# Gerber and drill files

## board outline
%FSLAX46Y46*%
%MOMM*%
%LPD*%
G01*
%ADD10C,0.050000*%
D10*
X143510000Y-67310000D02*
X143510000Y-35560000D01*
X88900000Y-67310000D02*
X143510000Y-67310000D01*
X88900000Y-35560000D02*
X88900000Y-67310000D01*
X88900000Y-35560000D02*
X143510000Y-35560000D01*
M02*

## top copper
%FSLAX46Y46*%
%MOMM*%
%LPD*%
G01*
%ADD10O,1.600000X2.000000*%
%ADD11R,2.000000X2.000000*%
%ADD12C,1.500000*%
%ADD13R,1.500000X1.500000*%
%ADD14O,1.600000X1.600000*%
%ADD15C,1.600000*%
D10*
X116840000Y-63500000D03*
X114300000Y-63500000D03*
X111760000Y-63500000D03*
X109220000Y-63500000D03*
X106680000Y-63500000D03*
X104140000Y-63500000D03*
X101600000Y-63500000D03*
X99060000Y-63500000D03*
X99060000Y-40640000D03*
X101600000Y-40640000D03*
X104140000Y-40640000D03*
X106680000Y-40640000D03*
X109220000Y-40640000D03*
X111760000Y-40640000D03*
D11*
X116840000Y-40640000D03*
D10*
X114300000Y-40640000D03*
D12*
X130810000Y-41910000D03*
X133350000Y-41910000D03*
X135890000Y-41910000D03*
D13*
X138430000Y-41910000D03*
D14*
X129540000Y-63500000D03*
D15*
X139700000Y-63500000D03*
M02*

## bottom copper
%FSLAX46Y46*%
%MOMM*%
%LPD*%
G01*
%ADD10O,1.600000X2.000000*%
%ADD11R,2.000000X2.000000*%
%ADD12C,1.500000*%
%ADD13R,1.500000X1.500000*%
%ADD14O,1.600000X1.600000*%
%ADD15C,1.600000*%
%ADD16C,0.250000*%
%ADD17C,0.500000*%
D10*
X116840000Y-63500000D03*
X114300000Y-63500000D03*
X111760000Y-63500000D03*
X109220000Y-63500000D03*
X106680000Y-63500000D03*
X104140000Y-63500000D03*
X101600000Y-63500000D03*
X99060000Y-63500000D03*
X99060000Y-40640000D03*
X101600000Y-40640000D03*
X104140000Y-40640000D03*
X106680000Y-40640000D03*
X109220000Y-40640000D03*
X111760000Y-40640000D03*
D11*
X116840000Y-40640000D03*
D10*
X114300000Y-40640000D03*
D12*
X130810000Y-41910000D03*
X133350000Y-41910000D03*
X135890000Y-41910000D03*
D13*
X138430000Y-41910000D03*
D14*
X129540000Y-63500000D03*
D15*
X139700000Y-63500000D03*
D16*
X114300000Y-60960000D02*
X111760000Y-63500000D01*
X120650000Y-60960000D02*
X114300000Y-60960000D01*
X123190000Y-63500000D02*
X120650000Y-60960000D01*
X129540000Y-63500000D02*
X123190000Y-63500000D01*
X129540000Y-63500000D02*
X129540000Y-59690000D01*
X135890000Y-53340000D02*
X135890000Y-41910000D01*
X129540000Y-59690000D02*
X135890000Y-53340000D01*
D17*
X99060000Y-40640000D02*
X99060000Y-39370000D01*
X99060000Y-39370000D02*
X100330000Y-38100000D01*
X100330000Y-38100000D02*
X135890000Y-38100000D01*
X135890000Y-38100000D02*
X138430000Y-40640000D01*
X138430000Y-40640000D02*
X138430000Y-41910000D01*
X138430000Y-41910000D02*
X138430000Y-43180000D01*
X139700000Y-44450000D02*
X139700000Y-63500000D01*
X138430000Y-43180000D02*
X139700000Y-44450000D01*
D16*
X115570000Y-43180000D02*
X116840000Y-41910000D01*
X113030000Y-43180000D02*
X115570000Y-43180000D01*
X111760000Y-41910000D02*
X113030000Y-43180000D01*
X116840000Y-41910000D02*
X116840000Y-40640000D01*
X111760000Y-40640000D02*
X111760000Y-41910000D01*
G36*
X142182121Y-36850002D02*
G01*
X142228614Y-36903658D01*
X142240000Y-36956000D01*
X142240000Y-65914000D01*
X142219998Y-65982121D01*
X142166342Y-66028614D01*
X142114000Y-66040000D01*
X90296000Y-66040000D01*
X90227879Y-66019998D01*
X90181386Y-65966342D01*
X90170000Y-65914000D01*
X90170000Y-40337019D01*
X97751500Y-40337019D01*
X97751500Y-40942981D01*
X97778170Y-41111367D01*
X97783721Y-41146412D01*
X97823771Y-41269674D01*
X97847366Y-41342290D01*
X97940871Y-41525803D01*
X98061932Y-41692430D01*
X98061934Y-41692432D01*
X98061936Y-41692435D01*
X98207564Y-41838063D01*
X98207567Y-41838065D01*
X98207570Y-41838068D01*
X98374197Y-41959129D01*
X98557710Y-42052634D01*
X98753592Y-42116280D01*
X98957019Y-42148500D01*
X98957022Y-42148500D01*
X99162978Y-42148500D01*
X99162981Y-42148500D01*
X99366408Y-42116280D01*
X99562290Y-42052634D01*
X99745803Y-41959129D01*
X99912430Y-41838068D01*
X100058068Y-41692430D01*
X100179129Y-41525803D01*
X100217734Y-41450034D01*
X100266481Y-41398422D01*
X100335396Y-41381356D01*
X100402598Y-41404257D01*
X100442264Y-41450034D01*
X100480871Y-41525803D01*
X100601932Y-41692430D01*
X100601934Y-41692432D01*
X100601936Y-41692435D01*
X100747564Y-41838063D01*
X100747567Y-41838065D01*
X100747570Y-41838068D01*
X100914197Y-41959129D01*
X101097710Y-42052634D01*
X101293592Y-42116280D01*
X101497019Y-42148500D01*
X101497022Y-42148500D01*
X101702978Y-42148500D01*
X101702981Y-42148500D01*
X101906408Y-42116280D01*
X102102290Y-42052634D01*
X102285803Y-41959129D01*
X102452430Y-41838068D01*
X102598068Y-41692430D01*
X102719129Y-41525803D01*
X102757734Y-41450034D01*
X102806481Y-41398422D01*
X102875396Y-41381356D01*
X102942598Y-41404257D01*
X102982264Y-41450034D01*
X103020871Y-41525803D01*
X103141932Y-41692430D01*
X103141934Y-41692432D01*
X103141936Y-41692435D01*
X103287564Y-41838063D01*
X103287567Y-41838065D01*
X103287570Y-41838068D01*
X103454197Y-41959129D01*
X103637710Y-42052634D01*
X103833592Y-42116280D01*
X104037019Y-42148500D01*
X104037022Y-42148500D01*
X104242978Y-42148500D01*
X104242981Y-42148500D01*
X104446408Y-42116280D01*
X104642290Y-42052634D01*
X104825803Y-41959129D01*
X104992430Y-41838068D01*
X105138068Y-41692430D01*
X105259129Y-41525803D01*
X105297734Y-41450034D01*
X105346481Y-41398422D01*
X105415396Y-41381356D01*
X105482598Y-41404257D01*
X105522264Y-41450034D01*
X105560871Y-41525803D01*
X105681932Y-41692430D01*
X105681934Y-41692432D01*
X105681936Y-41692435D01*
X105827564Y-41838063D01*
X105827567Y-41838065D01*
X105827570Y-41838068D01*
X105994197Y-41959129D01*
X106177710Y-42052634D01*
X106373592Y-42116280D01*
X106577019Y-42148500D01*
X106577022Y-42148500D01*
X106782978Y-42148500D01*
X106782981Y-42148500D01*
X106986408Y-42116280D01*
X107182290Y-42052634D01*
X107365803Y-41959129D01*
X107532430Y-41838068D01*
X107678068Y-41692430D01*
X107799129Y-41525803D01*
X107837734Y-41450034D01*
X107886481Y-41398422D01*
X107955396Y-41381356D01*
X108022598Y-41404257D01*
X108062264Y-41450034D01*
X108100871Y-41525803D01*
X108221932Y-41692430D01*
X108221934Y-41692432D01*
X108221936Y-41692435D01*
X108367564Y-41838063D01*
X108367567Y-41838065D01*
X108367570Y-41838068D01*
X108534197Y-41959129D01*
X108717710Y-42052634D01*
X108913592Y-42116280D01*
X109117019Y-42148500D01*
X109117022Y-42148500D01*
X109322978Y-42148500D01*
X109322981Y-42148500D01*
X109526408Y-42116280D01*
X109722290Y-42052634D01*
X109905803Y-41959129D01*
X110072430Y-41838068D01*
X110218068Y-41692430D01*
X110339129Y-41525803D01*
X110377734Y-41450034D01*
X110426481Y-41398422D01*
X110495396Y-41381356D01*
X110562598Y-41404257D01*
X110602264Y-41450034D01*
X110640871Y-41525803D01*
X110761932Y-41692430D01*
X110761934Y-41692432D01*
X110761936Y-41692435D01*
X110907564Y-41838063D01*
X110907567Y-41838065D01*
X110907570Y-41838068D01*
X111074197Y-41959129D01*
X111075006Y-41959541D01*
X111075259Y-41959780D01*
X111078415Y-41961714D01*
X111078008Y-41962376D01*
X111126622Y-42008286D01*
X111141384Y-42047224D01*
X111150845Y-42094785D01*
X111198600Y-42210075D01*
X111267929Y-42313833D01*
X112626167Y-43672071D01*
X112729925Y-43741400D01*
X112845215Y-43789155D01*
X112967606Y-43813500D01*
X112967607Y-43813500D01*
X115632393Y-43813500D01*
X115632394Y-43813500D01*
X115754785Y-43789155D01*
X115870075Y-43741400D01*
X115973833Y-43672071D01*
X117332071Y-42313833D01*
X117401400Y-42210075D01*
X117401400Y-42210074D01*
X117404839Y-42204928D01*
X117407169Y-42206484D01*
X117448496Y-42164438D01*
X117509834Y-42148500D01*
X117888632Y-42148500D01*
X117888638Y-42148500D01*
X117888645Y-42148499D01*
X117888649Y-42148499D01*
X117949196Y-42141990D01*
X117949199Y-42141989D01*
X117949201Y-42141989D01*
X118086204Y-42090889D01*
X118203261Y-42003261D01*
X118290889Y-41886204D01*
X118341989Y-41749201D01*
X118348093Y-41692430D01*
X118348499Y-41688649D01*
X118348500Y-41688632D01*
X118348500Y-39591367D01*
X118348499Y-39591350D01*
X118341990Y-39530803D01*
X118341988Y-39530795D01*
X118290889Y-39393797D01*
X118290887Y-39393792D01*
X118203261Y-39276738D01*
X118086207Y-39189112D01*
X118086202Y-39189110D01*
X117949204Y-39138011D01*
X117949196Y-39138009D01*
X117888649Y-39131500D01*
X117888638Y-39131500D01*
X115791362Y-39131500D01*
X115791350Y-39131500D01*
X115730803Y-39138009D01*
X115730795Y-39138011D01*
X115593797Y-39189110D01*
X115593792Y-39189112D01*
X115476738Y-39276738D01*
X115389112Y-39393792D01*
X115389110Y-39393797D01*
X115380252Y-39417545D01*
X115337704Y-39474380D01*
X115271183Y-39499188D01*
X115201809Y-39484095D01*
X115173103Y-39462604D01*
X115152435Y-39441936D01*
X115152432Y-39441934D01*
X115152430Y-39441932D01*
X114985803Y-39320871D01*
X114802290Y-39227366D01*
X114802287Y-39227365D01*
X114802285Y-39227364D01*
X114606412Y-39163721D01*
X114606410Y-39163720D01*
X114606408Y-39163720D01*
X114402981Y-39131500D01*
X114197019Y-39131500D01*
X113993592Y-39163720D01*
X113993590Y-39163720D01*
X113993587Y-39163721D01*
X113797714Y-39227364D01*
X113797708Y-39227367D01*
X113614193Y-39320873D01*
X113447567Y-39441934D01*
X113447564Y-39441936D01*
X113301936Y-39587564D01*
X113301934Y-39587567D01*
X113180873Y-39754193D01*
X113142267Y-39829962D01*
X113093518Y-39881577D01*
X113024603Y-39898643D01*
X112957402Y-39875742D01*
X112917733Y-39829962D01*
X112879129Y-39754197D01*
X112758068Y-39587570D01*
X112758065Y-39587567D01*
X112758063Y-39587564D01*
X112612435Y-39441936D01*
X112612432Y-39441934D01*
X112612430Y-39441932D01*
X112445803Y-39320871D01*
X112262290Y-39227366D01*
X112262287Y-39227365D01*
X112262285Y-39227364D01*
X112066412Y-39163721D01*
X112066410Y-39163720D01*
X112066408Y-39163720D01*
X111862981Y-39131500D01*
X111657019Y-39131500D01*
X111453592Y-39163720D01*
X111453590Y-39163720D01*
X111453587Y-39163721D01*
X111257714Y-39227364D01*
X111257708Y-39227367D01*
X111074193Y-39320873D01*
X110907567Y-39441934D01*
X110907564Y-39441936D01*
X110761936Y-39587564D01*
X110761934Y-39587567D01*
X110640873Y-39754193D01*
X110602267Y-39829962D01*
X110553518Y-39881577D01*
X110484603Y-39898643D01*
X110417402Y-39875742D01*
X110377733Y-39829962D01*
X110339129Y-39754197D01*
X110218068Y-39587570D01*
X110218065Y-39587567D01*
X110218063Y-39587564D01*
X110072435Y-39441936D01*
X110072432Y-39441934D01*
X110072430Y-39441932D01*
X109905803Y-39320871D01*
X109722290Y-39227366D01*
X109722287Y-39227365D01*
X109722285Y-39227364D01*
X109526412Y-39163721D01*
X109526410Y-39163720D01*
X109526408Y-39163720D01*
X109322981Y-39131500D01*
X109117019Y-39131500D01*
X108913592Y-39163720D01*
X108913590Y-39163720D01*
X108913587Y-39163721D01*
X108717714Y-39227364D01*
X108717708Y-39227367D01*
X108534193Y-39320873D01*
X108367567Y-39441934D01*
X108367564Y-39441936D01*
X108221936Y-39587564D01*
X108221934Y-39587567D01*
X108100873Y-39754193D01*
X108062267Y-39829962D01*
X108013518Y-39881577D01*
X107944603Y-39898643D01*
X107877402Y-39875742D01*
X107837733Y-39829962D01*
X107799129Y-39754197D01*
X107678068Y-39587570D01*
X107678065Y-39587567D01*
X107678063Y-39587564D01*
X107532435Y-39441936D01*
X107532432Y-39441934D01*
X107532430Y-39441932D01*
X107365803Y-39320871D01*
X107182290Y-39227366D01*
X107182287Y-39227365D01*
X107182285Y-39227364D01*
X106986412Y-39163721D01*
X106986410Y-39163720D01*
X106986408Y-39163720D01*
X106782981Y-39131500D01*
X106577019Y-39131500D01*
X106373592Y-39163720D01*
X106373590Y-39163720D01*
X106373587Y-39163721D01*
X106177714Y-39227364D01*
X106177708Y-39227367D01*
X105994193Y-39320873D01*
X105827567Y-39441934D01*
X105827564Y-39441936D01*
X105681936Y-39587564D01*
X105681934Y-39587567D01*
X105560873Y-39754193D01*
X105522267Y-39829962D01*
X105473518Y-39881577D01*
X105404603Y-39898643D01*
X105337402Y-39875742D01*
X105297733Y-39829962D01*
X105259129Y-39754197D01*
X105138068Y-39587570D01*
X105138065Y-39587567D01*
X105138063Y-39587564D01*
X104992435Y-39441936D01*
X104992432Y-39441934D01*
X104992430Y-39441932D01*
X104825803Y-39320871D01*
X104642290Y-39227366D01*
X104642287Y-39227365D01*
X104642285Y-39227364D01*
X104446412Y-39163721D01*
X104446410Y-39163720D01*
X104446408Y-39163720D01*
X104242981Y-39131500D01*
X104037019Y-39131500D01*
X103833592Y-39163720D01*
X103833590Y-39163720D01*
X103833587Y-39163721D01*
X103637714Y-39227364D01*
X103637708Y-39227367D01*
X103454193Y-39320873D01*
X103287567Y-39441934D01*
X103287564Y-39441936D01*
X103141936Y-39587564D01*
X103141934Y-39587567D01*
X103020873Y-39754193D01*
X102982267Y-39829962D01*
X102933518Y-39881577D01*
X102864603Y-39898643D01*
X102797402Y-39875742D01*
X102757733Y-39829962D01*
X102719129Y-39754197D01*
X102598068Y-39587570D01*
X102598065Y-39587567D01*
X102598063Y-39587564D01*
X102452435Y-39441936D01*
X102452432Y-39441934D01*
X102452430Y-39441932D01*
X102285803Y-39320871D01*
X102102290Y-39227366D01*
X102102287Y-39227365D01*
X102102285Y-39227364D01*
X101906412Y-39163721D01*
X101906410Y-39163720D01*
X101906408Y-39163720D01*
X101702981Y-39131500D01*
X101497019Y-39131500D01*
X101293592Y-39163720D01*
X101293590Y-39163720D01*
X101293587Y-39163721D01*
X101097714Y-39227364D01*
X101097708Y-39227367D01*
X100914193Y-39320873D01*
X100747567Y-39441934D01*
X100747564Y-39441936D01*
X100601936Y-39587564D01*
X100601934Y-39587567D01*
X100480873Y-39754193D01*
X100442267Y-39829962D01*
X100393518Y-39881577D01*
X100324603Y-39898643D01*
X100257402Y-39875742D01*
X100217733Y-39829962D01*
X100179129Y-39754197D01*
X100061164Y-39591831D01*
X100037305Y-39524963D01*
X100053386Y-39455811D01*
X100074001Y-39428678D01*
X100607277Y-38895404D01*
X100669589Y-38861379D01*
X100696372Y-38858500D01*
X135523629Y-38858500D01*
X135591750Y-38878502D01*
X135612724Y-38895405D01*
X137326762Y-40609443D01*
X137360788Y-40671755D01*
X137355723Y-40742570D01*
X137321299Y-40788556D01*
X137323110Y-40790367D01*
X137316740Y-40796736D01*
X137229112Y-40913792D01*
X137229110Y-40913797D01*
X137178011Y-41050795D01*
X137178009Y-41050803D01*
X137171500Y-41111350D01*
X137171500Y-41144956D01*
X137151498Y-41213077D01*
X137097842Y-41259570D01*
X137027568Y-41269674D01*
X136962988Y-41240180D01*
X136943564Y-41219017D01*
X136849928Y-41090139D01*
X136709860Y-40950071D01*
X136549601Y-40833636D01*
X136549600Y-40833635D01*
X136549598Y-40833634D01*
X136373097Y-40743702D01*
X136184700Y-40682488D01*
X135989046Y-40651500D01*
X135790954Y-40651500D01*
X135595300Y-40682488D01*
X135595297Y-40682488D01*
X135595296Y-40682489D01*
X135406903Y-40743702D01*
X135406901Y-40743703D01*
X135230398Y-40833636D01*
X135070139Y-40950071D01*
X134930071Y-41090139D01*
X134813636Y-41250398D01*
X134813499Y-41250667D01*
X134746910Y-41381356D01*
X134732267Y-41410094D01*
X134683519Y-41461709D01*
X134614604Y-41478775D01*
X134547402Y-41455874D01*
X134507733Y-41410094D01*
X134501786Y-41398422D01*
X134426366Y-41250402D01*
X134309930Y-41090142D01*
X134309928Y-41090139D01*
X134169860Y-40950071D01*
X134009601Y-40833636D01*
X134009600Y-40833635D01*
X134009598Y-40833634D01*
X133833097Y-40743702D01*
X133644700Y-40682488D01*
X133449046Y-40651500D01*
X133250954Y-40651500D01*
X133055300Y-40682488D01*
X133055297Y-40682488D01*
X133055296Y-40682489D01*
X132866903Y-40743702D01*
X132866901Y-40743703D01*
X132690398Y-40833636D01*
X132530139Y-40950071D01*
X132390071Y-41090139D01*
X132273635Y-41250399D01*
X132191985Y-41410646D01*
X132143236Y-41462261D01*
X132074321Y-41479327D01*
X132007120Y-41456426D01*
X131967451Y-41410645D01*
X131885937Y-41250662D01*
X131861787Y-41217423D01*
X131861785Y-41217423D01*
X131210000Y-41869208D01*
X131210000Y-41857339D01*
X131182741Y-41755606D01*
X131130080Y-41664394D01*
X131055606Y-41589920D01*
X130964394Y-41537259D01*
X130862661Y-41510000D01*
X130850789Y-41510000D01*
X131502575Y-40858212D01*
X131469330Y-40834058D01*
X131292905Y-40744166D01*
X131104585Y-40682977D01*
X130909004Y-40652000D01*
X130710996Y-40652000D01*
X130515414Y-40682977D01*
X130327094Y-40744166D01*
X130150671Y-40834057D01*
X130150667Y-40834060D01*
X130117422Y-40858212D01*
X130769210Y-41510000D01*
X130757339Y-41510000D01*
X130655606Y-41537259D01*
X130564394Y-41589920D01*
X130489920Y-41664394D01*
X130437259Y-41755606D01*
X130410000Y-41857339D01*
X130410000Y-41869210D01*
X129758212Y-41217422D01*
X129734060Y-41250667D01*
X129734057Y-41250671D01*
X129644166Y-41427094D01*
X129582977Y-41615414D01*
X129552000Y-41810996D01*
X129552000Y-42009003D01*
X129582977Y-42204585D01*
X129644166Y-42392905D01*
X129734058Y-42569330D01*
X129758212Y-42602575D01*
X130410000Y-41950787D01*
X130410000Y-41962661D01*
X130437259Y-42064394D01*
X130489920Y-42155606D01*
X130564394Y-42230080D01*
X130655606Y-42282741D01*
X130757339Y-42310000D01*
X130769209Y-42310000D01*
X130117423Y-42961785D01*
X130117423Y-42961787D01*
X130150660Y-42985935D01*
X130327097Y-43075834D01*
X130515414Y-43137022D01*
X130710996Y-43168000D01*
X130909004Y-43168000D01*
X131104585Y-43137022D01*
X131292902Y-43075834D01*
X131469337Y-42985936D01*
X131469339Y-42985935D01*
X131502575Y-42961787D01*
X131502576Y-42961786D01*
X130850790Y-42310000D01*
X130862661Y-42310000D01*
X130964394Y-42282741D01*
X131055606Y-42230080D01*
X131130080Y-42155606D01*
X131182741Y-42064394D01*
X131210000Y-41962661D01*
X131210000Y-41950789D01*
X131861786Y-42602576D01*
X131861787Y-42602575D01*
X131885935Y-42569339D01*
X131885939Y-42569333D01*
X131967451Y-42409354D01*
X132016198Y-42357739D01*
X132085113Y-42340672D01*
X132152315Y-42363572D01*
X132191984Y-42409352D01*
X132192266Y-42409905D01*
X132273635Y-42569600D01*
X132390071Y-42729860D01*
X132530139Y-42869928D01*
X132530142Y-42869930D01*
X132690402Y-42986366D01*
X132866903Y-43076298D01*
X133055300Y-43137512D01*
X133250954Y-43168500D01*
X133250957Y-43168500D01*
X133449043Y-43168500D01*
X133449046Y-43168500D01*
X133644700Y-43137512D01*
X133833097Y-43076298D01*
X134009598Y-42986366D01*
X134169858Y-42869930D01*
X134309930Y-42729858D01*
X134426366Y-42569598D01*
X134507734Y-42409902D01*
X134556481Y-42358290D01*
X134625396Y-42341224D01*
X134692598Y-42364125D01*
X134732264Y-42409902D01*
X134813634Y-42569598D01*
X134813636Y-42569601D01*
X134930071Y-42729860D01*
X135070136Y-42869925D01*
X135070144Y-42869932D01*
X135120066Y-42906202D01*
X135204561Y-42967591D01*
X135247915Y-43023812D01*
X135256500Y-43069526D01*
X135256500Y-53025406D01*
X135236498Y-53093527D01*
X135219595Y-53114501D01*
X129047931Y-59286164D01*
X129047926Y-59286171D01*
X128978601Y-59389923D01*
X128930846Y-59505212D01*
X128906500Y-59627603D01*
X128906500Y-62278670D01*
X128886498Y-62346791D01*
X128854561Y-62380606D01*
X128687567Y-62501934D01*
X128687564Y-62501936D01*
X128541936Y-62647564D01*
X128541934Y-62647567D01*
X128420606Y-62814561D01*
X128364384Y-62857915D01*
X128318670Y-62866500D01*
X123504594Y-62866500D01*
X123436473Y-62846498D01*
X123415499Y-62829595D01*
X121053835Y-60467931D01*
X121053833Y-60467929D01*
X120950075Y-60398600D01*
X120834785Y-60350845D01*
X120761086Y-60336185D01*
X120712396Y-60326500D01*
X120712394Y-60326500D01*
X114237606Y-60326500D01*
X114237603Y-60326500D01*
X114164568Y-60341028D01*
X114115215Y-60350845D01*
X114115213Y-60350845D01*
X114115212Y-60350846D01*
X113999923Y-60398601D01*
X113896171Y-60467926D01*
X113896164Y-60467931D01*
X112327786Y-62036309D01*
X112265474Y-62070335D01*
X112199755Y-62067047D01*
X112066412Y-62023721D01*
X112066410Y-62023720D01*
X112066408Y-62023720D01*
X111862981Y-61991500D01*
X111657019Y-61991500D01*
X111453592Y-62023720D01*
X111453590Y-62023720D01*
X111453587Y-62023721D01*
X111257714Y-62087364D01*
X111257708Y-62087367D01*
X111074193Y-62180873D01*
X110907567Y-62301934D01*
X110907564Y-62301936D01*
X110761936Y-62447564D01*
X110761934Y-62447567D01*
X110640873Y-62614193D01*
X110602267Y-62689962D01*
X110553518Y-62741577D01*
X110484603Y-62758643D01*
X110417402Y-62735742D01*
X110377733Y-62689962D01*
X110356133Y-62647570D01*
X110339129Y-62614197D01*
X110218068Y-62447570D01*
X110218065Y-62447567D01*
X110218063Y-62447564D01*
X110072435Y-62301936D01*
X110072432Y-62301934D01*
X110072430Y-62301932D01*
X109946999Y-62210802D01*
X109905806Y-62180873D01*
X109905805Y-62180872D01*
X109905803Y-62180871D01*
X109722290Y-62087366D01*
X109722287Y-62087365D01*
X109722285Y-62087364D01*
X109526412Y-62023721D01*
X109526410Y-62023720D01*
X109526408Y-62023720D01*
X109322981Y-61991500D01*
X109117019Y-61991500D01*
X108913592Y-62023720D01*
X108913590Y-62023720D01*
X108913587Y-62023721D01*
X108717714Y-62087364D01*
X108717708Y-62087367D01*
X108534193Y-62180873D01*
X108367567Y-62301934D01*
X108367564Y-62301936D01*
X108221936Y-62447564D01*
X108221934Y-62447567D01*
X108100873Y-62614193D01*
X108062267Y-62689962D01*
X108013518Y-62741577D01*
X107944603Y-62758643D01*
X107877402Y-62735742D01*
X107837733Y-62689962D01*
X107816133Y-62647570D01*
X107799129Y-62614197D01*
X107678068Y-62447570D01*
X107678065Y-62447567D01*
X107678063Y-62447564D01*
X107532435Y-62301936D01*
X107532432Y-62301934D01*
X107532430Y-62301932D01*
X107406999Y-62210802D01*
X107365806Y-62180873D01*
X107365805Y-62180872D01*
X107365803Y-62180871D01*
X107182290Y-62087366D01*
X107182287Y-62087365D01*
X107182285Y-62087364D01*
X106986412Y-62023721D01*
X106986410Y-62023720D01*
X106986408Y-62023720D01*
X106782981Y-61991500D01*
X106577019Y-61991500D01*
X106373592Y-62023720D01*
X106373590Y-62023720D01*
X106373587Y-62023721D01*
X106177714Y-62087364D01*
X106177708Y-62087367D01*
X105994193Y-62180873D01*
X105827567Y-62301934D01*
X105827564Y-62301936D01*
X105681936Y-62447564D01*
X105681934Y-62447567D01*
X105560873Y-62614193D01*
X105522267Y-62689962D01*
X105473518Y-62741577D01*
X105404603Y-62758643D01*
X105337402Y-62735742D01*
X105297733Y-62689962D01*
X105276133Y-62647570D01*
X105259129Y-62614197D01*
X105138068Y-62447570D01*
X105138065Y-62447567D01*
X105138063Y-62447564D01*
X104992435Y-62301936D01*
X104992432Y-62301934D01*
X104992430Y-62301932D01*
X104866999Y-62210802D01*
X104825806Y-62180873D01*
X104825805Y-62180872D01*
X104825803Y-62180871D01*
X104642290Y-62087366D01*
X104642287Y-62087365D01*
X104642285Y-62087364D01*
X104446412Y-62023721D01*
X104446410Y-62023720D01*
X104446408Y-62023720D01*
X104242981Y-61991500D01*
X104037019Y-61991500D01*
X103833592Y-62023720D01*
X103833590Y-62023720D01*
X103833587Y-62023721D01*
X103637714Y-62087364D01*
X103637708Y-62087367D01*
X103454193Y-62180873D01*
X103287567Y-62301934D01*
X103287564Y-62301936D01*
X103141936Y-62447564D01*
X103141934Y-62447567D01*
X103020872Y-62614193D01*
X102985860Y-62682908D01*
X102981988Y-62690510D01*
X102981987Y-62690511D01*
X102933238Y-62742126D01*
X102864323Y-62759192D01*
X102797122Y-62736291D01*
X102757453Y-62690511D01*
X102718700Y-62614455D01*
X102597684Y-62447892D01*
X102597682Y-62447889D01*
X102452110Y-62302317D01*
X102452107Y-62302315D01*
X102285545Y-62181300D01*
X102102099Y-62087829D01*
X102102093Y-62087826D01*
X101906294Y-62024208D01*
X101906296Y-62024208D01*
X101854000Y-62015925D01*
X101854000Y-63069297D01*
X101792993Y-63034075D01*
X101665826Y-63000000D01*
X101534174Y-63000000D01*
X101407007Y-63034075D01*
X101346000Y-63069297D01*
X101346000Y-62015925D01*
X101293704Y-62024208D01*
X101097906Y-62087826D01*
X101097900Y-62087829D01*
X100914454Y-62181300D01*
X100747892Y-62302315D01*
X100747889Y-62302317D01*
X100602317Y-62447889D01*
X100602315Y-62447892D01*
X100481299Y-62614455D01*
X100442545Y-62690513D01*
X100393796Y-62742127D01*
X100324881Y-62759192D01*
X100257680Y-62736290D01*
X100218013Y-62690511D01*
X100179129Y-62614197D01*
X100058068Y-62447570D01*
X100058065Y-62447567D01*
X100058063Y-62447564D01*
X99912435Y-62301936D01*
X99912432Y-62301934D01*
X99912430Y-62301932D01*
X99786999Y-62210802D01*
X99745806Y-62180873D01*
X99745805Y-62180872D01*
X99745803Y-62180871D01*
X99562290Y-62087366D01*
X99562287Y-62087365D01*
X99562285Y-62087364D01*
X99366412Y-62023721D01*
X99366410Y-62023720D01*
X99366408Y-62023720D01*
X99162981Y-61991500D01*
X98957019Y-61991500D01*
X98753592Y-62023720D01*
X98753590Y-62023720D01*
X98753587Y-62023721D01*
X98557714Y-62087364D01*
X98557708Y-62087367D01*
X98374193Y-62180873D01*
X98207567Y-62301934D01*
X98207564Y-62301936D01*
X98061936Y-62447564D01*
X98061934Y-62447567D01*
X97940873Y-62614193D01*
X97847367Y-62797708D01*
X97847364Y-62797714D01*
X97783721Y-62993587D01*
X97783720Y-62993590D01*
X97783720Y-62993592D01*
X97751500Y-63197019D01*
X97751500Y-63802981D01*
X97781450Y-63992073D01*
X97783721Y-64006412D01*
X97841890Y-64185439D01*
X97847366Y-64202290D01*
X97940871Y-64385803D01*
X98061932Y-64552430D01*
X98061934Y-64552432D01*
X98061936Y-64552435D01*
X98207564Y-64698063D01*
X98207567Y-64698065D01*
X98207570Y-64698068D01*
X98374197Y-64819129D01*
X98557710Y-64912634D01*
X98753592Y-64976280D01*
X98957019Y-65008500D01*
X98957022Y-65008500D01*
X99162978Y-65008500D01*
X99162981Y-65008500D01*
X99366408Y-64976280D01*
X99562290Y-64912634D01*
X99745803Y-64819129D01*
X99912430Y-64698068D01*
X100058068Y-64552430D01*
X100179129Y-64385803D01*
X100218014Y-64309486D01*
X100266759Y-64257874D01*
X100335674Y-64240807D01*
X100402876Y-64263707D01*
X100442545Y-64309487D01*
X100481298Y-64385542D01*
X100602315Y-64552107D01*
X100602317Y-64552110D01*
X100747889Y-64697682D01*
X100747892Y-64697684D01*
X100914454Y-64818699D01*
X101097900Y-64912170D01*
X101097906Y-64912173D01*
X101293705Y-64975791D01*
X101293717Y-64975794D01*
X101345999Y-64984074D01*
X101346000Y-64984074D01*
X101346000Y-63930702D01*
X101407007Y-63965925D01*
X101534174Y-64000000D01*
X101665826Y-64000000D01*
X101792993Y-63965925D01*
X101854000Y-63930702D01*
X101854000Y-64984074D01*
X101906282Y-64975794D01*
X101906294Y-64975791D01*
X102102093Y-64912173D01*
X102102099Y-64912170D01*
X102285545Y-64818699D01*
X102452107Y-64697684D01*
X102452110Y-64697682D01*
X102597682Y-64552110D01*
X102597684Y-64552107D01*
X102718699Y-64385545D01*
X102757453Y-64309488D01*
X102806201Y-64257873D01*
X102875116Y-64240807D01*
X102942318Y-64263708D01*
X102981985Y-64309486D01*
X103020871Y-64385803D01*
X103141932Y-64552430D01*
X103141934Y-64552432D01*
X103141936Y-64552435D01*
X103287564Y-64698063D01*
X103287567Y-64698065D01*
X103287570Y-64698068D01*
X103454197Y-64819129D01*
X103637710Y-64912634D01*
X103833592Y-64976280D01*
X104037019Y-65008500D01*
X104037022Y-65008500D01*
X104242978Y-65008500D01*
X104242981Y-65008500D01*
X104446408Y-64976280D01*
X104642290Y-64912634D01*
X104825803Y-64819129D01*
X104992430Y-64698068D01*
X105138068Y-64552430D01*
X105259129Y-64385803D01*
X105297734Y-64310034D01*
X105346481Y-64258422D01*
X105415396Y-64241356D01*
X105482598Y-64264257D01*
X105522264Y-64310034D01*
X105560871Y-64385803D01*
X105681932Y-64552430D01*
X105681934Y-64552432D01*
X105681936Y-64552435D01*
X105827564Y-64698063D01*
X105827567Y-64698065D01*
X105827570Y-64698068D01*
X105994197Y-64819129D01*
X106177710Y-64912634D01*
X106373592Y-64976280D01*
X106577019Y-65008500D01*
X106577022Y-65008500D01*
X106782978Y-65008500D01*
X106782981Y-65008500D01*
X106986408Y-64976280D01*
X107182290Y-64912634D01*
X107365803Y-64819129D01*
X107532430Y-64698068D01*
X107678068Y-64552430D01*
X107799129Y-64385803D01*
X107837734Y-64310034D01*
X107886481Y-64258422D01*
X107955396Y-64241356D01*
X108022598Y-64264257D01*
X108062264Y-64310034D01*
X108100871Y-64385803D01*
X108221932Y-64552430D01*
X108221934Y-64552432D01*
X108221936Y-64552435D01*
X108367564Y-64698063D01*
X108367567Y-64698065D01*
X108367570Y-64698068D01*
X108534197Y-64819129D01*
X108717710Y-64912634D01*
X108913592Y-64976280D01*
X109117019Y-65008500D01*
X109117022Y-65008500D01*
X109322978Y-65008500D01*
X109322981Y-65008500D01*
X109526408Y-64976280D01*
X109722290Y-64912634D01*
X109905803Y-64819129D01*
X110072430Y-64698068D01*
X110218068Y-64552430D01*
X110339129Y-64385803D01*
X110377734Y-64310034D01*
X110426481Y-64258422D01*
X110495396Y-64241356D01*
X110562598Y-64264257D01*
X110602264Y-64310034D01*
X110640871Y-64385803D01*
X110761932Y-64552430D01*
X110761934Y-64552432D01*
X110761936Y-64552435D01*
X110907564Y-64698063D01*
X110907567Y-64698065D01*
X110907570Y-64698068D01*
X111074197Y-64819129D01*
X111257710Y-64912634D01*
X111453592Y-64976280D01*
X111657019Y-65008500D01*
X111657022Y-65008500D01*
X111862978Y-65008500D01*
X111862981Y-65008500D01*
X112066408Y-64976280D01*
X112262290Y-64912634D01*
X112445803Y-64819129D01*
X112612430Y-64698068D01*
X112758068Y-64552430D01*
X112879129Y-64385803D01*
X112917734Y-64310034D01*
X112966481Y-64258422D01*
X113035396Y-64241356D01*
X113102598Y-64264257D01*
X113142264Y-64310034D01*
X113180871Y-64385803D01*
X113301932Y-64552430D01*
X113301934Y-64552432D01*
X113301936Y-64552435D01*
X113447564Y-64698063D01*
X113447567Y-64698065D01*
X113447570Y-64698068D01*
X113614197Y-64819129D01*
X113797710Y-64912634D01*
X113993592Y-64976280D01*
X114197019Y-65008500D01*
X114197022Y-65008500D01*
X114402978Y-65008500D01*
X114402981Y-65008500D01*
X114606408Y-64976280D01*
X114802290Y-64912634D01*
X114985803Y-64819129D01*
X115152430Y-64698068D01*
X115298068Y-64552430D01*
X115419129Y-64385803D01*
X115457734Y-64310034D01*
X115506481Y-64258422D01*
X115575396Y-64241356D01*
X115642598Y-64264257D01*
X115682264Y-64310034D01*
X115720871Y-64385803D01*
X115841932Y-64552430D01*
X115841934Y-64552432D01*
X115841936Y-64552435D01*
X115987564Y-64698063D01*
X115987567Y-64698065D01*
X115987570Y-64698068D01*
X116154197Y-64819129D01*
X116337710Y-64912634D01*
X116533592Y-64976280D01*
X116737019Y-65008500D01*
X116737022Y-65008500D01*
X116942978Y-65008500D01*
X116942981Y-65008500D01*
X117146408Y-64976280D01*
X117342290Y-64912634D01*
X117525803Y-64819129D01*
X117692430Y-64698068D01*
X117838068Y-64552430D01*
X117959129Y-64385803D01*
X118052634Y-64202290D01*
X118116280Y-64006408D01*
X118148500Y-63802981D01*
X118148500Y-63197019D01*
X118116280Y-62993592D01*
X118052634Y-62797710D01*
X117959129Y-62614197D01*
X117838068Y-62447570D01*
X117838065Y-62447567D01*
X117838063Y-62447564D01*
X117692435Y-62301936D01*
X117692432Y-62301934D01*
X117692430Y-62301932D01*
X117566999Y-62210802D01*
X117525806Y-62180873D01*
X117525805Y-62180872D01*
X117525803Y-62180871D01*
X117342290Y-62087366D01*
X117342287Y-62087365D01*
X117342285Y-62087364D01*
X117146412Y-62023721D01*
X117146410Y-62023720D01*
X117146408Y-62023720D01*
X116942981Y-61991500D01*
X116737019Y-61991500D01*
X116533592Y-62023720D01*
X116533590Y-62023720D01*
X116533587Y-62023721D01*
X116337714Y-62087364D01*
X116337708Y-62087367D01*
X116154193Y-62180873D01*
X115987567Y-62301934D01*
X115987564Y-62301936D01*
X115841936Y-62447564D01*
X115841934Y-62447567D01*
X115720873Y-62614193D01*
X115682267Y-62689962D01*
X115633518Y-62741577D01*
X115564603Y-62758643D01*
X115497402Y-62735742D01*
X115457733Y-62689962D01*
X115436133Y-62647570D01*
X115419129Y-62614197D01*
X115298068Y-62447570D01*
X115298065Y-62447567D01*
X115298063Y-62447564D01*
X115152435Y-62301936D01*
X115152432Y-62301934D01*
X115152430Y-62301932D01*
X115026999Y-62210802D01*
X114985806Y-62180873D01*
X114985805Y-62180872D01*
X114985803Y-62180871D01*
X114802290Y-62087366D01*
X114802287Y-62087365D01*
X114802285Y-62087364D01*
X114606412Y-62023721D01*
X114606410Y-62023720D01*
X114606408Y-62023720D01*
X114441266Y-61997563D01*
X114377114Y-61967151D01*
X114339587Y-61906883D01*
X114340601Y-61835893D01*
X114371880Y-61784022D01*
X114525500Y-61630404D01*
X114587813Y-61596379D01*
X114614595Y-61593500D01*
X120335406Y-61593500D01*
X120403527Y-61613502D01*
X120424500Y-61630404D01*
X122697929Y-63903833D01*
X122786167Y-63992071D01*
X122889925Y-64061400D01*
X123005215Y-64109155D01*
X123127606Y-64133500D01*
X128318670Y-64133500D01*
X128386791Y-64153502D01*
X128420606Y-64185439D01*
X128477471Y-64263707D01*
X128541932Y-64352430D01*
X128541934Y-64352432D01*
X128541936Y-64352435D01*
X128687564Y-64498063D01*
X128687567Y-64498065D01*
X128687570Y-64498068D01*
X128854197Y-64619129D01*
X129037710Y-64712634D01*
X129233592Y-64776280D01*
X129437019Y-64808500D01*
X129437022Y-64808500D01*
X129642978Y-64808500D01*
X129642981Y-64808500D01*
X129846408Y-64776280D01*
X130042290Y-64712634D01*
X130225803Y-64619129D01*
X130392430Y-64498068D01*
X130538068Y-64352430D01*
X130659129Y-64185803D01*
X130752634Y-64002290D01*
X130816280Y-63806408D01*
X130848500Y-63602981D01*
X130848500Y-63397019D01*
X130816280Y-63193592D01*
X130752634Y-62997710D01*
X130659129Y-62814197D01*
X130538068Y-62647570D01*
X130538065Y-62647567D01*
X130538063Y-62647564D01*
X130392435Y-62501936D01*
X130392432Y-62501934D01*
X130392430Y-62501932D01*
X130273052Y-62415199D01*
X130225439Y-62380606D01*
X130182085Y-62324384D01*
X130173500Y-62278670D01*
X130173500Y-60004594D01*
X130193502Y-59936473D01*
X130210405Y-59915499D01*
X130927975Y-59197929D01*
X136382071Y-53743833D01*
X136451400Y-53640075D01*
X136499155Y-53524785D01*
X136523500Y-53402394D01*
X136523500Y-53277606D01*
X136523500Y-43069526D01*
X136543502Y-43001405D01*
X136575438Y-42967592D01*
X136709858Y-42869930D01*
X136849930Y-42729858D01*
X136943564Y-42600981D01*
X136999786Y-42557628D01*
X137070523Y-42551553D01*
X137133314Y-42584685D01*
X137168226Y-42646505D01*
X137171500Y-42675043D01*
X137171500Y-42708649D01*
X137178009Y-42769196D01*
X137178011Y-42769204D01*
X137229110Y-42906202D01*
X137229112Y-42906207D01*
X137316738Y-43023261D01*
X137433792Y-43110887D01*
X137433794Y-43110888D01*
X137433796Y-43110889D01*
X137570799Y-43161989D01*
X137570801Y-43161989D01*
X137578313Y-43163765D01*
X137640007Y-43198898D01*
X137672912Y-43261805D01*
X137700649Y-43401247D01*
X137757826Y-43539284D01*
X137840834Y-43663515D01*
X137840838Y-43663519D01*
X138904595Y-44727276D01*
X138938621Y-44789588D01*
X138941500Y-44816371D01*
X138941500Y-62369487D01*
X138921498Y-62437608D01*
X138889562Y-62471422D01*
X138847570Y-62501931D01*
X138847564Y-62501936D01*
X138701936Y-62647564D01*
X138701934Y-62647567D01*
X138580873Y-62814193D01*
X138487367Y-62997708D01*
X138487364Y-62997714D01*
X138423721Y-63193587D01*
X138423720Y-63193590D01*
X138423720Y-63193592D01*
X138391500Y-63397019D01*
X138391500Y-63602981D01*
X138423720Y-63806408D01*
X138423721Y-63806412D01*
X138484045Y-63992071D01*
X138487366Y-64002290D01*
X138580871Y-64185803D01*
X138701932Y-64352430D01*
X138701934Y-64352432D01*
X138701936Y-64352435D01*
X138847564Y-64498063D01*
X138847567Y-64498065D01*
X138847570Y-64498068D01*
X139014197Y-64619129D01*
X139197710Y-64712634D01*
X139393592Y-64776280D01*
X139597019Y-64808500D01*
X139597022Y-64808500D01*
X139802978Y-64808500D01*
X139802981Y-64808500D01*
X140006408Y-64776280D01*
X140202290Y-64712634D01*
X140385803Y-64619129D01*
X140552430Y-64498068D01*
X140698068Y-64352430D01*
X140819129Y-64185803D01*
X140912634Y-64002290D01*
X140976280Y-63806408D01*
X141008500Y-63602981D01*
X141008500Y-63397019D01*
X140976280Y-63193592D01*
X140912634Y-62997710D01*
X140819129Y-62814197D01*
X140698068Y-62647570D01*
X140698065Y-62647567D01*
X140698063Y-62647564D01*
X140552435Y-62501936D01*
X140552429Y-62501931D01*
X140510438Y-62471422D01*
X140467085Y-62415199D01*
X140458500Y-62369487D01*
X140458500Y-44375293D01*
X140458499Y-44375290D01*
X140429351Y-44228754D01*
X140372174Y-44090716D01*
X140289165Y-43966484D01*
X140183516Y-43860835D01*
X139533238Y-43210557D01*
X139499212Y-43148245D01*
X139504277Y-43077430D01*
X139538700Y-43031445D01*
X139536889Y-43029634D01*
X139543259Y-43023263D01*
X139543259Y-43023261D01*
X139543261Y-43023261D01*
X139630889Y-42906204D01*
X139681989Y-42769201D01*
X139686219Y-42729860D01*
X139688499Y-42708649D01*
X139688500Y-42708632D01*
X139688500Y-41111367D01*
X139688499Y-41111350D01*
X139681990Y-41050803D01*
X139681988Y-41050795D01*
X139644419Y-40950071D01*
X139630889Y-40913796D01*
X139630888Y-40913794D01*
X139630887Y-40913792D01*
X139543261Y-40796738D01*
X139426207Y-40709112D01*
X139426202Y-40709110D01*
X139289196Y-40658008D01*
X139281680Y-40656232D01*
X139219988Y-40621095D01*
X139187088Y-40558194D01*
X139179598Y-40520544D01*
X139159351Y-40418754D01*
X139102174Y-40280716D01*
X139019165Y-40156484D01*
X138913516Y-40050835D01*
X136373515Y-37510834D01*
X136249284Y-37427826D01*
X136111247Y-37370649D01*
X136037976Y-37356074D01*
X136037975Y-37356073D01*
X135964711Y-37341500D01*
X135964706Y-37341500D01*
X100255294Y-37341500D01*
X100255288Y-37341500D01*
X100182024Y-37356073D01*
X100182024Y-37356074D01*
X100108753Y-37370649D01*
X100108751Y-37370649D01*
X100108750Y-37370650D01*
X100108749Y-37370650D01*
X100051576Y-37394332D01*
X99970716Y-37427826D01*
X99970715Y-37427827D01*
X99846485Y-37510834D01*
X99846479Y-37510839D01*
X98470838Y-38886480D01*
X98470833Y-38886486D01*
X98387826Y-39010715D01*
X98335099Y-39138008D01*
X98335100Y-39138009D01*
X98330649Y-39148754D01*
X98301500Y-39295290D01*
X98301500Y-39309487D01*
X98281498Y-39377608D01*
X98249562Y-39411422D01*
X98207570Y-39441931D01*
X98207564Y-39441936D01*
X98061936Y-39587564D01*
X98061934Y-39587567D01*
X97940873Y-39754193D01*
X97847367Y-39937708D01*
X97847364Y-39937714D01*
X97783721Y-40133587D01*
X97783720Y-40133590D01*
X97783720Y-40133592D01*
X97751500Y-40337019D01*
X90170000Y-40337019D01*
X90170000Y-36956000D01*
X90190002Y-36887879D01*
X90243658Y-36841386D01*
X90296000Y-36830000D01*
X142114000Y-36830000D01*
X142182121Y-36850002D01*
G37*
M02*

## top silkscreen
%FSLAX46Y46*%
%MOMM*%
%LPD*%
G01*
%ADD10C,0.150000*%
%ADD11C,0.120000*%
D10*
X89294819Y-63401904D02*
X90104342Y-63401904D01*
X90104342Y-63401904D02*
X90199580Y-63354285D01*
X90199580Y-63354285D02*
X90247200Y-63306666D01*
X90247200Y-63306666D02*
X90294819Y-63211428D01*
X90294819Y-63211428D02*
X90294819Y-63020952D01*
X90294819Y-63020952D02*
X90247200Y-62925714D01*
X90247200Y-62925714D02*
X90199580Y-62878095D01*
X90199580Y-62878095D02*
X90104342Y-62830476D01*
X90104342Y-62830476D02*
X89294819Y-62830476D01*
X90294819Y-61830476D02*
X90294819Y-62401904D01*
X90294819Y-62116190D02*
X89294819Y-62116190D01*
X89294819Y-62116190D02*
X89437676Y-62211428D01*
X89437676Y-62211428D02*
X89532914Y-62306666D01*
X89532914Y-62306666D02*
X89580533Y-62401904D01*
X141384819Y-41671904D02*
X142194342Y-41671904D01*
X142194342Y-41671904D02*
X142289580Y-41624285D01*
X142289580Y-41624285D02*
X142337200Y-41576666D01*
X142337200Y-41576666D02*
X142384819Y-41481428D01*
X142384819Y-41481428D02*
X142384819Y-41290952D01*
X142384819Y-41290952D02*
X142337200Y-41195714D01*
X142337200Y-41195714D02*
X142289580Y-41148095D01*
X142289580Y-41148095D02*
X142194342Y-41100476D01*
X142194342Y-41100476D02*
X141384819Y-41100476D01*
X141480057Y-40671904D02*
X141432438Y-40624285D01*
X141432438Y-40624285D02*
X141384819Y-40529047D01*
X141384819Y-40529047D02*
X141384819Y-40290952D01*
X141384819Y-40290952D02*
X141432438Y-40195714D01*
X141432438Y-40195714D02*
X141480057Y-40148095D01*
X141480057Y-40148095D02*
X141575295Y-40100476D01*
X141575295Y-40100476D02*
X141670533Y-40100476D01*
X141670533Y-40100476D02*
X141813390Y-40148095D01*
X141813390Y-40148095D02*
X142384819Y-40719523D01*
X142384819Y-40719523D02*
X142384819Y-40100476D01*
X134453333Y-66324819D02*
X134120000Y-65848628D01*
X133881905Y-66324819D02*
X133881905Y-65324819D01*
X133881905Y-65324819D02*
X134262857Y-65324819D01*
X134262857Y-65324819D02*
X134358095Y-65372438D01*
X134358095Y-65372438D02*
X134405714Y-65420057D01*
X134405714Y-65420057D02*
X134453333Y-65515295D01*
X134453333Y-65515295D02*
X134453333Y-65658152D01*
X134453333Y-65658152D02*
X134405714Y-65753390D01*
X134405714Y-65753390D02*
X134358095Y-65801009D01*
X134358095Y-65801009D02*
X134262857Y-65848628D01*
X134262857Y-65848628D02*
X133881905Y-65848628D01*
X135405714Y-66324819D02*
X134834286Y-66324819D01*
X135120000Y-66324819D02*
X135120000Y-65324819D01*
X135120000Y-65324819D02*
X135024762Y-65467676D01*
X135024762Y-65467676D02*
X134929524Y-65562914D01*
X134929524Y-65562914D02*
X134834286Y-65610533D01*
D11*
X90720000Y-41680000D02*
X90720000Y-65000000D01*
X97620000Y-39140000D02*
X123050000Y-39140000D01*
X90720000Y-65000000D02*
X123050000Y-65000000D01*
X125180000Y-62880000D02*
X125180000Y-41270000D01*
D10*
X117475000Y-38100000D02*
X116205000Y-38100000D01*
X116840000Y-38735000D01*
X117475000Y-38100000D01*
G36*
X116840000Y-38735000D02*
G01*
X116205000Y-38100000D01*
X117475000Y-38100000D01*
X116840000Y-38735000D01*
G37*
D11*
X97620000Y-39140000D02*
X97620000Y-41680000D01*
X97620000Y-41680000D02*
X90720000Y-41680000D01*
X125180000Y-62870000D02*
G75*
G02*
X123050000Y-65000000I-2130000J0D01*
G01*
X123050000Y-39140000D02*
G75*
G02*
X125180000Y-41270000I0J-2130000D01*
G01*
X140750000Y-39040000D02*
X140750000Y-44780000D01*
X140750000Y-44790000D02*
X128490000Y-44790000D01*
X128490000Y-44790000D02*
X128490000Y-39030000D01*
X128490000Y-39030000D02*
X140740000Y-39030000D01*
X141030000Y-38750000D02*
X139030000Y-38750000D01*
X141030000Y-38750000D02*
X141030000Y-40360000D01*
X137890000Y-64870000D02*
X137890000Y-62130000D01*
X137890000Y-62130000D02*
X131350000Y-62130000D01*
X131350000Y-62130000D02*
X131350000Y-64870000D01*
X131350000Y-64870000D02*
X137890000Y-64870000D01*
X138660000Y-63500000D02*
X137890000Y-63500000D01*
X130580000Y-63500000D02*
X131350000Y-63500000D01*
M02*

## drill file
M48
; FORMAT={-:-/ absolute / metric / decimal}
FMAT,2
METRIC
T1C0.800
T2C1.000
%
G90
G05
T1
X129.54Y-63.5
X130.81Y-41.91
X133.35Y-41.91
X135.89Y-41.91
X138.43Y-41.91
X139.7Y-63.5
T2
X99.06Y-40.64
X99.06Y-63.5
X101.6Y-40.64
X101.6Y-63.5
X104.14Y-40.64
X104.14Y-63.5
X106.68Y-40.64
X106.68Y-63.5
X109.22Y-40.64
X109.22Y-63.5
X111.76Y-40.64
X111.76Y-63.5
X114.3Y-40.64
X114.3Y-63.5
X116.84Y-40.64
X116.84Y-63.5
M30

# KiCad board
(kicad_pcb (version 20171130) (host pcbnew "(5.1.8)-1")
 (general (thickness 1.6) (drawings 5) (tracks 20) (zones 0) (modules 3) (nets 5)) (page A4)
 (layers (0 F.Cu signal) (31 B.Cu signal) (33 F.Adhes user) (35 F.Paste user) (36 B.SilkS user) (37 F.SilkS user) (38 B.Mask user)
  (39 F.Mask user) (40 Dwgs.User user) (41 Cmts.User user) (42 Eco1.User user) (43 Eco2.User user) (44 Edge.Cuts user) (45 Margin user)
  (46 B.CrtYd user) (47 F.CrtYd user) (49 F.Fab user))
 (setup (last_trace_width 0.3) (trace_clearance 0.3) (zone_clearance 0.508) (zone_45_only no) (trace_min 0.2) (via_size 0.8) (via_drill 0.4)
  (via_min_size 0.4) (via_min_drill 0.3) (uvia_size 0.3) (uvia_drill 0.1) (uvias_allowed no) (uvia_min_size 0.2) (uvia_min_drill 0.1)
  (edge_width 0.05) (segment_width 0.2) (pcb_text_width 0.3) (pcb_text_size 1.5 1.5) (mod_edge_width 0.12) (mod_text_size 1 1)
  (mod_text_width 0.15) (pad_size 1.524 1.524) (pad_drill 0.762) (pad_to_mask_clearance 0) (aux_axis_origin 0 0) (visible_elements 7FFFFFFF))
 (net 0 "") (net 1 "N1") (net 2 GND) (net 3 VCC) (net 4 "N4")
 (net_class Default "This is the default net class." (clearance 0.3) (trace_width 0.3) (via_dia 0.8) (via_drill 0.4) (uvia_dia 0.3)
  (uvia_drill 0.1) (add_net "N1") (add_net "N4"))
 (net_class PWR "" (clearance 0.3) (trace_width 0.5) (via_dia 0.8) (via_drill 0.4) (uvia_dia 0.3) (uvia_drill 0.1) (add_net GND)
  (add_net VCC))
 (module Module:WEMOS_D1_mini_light (layer F.Cu) (at 116.84 40.64 270)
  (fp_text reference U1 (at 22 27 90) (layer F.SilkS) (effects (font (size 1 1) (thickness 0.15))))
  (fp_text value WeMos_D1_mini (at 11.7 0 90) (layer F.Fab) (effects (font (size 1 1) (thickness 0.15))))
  (fp_line (start 1.04 26.12) (end 24.36 26.12) (layer F.SilkS) (width 0.12))
  (fp_line (start -1.5 19.22) (end -1.5 -6.21) (layer F.SilkS) (width 0.12))
  (fp_line (start 24.36 26.12) (end 24.36 -6.21) (layer F.SilkS) (width 0.12))
  (fp_line (start 22.24 -8.34) (end 0.63 -8.34) (layer F.SilkS) (width 0.12))
  (fp_poly (pts (xy -2.54 -0.635) (xy -2.54 0.635) (xy -1.905 0)) (layer F.SilkS) (width 0.15))
  (fp_line (start -1.5 19.22) (end 1.04 19.22) (layer F.SilkS) (width 0.12))
  (fp_line (start 1.04 19.22) (end 1.04 26.12) (layer F.SilkS) (width 0.12))
  (fp_arc (start 22.23 -6.21) (end 24.36 -6.21) (angle -90) (layer F.SilkS) (width 0.12))
  (fp_arc (start 0.63 -6.21) (end 0.63 -8.34) (angle -90) (layer F.SilkS) (width 0.12))
  (pad 16 thru_hole oval (at 22.86 0 270) (size 2 1.6) (drill 1) (layers *.Cu *.Mask))
  (pad 15 thru_hole oval (at 22.86 2.54 270) (size 2 1.6) (drill 1) (layers *.Cu *.Mask))
  (pad 14 thru_hole oval (at 22.86 5.08 270) (size 2 1.6) (drill 1) (layers *.Cu *.Mask) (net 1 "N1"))
  (pad 13 thru_hole oval (at 22.86 7.62 270) (size 2 1.6) (drill 1) (layers *.Cu *.Mask))
  (pad 12 thru_hole oval (at 22.86 10.16 270) (size 2 1.6) (drill 1) (layers *.Cu *.Mask))
  (pad 11 thru_hole oval (at 22.86 12.7 270) (size 2 1.6) (drill 1) (layers *.Cu *.Mask))
  (pad 10 thru_hole oval (at 22.86 15.24 270) (size 2 1.6) (drill 1) (layers *.Cu *.Mask) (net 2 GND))
  (pad 9 thru_hole oval (at 22.86 17.78 270) (size 2 1.6) (drill 1) (layers *.Cu *.Mask))
  (pad 8 thru_hole oval (at 0 17.78 270) (size 2 1.6) (drill 1) (layers *.Cu *.Mask) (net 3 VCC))
  (pad 7 thru_hole oval (at 0 15.24 270) (size 2 1.6) (drill 1) (layers *.Cu *.Mask))
  (pad 6 thru_hole oval (at 0 12.7 270) (size 2 1.6) (drill 1) (layers *.Cu *.Mask))
  (pad 5 thru_hole oval (at 0 10.16 270) (size 2 1.6) (drill 1) (layers *.Cu *.Mask))
  (pad 4 thru_hole oval (at 0 7.62 270) (size 2 1.6) (drill 1) (layers *.Cu *.Mask))
  (pad 3 thru_hole oval (at 0 5.08 270) (size 2 1.6) (drill 1) (layers *.Cu *.Mask) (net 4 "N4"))
  (pad 1 thru_hole rect (at 0 0 270) (size 2 2) (drill 1) (layers *.Cu *.Mask) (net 4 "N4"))
  (pad 2 thru_hole oval (at 0 2.54 270) (size 2 1.6) (drill 1) (layers *.Cu *.Mask)))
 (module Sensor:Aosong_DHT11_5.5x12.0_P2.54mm (layer F.Cu) (at 138.43 41.91 270)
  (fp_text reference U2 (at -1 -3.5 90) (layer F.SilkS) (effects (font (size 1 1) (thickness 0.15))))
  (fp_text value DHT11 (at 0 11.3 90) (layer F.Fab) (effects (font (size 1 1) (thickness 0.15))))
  (fp_line (start -2.87 -2.32) (end 2.87 -2.32) (layer F.SilkS) (width 0.12))
  (fp_line (start 2.88 -2.32) (end 2.88 9.94) (layer F.SilkS) (width 0.12))
  (fp_line (start 2.88 9.94) (end -2.88 9.94) (layer F.SilkS) (width 0.12))
  (fp_line (start -2.88 9.94) (end -2.88 -2.31) (layer F.SilkS) (width 0.12))
  (fp_line (start -3.16 -2.6) (end -3.16 -0.6) (layer F.SilkS) (width 0.12))
  (fp_line (start -3.16 -2.6) (end -1.55 -2.6) (layer F.SilkS) (width 0.12))
  (pad 4 thru_hole circle (at 0 7.62 270) (size 1.5 1.5) (drill 0.8) (layers *.Cu *.Mask) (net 2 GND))
  (pad 3 thru_hole circle (at 0 5.08 270) (size 1.5 1.5) (drill 0.8) (layers *.Cu *.Mask))
  (pad 2 thru_hole circle (at 0 2.54 270) (size 1.5 1.5) (drill 0.8) (layers *.Cu *.Mask) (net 1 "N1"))
  (pad 1 thru_hole rect (at 0 0 270) (size 1.5 1.5) (drill 0.8) (layers *.Cu *.Mask) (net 3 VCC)))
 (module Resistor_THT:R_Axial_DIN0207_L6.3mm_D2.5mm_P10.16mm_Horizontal (layer F.Cu) (at 139.7 63.5 180)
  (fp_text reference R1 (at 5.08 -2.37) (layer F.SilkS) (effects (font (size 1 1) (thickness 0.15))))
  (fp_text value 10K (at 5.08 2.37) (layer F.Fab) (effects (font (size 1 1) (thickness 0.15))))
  (fp_line (start 1.81 -1.37) (end 1.81 1.37) (layer F.SilkS) (width 0.12))
  (fp_line (start 1.81 1.37) (end 8.35 1.37) (layer F.SilkS) (width 0.12))
  (fp_line (start 8.35 1.37) (end 8.35 -1.37) (layer F.SilkS) (width 0.12))
  (fp_line (start 8.35 -1.37) (end 1.81 -1.37) (layer F.SilkS) (width 0.12))
  (fp_line (start 1.04 0) (end 1.81 0) (layer F.SilkS) (width 0.12))
  (fp_line (start 9.12 0) (end 8.35 0) (layer F.SilkS) (width 0.12))
  (pad 2 thru_hole oval (at 10.16 0 180) (size 1.6 1.6) (drill 0.8) (layers *.Cu *.Mask) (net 1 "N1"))
  (pad 1 thru_hole circle (at 0 0 180) (size 1.6 1.6) (drill 0.8) (layers *.Cu *.Mask) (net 3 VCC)))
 (gr_line (start 143.51 67.31) (end 143.51 35.56) (layer Edge.Cuts) (width 0.05))
 (gr_line (start 88.9 67.31) (end 143.51 67.31) (layer Edge.Cuts) (width 0.05))
 (gr_line (start 88.9 35.56) (end 88.9 67.31) (layer Edge.Cuts) (width 0.05))
 (gr_line (start 88.9 35.56) (end 143.51 35.56) (layer Edge.Cuts) (width 0.05))
 (segment (start 114.3 60.96) (end 111.76 63.5) (width 0.25) (layer B.Cu) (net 1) (status 20))
 (segment (start 120.65 60.96) (end 114.3 60.96) (width 0.25) (layer B.Cu) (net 1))
 (segment (start 123.19 63.5) (end 120.65 60.96) (width 0.25) (layer B.Cu) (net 1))
 (segment (start 129.54 63.5) (end 123.19 63.5) (width 0.25) (layer B.Cu) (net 1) (status 10))
 (segment (start 129.54 63.5) (end 129.54 59.69) (width 0.25) (layer B.Cu) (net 1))
 (segment (start 135.89 53.34) (end 135.89 41.91) (width 0.25) (layer B.Cu) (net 1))
 (segment (start 129.54 59.69) (end 135.89 53.34) (width 0.25) (layer B.Cu) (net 1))
 (segment (start 99.06 40.64) (end 99.06 39.37) (width 0.5) (layer B.Cu) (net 3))
 (segment (start 99.06 39.37) (end 100.33 38.1) (width 0.5) (layer B.Cu) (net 3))
 (segment (start 100.33 38.1) (end 135.89 38.1) (width 0.5) (layer B.Cu) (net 3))
 (segment (start 135.89 38.1) (end 138.43 40.64) (width 0.5) (layer B.Cu) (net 3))
 (segment (start 138.43 40.64) (end 138.43 41.91) (width 0.5) (layer B.Cu) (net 3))
 (segment (start 138.43 41.91) (end 138.43 43.18) (width 0.5) (layer B.Cu) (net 3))
 (segment (start 139.7 44.45) (end 139.7 63.5) (width 0.5) (layer B.Cu) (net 3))
 (segment (start 138.43 43.18) (end 139.7 44.45) (width 0.5) (layer B.Cu) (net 3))
 (segment (start 115.57 43.18) (end 116.84 41.91) (width 0.25) (layer B.Cu) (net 4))
 (segment (start 113.03 43.18) (end 115.57 43.18) (width 0.25) (layer B.Cu) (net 4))
 (segment (start 111.76 41.91) (end 113.03 43.18) (width 0.25) (layer B.Cu) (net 4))
 (segment (start 116.84 41.91) (end 116.84 40.64) (width 0.25) (layer B.Cu) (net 4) (status 20))
 (segment (start 111.76 40.64) (end 111.76 41.91) (width 0.25) (layer B.Cu) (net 4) (status 10))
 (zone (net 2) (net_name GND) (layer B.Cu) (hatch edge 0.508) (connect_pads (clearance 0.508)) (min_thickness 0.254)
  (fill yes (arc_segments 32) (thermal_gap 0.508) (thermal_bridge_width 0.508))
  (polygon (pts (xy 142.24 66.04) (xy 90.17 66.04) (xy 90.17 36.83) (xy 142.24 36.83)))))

